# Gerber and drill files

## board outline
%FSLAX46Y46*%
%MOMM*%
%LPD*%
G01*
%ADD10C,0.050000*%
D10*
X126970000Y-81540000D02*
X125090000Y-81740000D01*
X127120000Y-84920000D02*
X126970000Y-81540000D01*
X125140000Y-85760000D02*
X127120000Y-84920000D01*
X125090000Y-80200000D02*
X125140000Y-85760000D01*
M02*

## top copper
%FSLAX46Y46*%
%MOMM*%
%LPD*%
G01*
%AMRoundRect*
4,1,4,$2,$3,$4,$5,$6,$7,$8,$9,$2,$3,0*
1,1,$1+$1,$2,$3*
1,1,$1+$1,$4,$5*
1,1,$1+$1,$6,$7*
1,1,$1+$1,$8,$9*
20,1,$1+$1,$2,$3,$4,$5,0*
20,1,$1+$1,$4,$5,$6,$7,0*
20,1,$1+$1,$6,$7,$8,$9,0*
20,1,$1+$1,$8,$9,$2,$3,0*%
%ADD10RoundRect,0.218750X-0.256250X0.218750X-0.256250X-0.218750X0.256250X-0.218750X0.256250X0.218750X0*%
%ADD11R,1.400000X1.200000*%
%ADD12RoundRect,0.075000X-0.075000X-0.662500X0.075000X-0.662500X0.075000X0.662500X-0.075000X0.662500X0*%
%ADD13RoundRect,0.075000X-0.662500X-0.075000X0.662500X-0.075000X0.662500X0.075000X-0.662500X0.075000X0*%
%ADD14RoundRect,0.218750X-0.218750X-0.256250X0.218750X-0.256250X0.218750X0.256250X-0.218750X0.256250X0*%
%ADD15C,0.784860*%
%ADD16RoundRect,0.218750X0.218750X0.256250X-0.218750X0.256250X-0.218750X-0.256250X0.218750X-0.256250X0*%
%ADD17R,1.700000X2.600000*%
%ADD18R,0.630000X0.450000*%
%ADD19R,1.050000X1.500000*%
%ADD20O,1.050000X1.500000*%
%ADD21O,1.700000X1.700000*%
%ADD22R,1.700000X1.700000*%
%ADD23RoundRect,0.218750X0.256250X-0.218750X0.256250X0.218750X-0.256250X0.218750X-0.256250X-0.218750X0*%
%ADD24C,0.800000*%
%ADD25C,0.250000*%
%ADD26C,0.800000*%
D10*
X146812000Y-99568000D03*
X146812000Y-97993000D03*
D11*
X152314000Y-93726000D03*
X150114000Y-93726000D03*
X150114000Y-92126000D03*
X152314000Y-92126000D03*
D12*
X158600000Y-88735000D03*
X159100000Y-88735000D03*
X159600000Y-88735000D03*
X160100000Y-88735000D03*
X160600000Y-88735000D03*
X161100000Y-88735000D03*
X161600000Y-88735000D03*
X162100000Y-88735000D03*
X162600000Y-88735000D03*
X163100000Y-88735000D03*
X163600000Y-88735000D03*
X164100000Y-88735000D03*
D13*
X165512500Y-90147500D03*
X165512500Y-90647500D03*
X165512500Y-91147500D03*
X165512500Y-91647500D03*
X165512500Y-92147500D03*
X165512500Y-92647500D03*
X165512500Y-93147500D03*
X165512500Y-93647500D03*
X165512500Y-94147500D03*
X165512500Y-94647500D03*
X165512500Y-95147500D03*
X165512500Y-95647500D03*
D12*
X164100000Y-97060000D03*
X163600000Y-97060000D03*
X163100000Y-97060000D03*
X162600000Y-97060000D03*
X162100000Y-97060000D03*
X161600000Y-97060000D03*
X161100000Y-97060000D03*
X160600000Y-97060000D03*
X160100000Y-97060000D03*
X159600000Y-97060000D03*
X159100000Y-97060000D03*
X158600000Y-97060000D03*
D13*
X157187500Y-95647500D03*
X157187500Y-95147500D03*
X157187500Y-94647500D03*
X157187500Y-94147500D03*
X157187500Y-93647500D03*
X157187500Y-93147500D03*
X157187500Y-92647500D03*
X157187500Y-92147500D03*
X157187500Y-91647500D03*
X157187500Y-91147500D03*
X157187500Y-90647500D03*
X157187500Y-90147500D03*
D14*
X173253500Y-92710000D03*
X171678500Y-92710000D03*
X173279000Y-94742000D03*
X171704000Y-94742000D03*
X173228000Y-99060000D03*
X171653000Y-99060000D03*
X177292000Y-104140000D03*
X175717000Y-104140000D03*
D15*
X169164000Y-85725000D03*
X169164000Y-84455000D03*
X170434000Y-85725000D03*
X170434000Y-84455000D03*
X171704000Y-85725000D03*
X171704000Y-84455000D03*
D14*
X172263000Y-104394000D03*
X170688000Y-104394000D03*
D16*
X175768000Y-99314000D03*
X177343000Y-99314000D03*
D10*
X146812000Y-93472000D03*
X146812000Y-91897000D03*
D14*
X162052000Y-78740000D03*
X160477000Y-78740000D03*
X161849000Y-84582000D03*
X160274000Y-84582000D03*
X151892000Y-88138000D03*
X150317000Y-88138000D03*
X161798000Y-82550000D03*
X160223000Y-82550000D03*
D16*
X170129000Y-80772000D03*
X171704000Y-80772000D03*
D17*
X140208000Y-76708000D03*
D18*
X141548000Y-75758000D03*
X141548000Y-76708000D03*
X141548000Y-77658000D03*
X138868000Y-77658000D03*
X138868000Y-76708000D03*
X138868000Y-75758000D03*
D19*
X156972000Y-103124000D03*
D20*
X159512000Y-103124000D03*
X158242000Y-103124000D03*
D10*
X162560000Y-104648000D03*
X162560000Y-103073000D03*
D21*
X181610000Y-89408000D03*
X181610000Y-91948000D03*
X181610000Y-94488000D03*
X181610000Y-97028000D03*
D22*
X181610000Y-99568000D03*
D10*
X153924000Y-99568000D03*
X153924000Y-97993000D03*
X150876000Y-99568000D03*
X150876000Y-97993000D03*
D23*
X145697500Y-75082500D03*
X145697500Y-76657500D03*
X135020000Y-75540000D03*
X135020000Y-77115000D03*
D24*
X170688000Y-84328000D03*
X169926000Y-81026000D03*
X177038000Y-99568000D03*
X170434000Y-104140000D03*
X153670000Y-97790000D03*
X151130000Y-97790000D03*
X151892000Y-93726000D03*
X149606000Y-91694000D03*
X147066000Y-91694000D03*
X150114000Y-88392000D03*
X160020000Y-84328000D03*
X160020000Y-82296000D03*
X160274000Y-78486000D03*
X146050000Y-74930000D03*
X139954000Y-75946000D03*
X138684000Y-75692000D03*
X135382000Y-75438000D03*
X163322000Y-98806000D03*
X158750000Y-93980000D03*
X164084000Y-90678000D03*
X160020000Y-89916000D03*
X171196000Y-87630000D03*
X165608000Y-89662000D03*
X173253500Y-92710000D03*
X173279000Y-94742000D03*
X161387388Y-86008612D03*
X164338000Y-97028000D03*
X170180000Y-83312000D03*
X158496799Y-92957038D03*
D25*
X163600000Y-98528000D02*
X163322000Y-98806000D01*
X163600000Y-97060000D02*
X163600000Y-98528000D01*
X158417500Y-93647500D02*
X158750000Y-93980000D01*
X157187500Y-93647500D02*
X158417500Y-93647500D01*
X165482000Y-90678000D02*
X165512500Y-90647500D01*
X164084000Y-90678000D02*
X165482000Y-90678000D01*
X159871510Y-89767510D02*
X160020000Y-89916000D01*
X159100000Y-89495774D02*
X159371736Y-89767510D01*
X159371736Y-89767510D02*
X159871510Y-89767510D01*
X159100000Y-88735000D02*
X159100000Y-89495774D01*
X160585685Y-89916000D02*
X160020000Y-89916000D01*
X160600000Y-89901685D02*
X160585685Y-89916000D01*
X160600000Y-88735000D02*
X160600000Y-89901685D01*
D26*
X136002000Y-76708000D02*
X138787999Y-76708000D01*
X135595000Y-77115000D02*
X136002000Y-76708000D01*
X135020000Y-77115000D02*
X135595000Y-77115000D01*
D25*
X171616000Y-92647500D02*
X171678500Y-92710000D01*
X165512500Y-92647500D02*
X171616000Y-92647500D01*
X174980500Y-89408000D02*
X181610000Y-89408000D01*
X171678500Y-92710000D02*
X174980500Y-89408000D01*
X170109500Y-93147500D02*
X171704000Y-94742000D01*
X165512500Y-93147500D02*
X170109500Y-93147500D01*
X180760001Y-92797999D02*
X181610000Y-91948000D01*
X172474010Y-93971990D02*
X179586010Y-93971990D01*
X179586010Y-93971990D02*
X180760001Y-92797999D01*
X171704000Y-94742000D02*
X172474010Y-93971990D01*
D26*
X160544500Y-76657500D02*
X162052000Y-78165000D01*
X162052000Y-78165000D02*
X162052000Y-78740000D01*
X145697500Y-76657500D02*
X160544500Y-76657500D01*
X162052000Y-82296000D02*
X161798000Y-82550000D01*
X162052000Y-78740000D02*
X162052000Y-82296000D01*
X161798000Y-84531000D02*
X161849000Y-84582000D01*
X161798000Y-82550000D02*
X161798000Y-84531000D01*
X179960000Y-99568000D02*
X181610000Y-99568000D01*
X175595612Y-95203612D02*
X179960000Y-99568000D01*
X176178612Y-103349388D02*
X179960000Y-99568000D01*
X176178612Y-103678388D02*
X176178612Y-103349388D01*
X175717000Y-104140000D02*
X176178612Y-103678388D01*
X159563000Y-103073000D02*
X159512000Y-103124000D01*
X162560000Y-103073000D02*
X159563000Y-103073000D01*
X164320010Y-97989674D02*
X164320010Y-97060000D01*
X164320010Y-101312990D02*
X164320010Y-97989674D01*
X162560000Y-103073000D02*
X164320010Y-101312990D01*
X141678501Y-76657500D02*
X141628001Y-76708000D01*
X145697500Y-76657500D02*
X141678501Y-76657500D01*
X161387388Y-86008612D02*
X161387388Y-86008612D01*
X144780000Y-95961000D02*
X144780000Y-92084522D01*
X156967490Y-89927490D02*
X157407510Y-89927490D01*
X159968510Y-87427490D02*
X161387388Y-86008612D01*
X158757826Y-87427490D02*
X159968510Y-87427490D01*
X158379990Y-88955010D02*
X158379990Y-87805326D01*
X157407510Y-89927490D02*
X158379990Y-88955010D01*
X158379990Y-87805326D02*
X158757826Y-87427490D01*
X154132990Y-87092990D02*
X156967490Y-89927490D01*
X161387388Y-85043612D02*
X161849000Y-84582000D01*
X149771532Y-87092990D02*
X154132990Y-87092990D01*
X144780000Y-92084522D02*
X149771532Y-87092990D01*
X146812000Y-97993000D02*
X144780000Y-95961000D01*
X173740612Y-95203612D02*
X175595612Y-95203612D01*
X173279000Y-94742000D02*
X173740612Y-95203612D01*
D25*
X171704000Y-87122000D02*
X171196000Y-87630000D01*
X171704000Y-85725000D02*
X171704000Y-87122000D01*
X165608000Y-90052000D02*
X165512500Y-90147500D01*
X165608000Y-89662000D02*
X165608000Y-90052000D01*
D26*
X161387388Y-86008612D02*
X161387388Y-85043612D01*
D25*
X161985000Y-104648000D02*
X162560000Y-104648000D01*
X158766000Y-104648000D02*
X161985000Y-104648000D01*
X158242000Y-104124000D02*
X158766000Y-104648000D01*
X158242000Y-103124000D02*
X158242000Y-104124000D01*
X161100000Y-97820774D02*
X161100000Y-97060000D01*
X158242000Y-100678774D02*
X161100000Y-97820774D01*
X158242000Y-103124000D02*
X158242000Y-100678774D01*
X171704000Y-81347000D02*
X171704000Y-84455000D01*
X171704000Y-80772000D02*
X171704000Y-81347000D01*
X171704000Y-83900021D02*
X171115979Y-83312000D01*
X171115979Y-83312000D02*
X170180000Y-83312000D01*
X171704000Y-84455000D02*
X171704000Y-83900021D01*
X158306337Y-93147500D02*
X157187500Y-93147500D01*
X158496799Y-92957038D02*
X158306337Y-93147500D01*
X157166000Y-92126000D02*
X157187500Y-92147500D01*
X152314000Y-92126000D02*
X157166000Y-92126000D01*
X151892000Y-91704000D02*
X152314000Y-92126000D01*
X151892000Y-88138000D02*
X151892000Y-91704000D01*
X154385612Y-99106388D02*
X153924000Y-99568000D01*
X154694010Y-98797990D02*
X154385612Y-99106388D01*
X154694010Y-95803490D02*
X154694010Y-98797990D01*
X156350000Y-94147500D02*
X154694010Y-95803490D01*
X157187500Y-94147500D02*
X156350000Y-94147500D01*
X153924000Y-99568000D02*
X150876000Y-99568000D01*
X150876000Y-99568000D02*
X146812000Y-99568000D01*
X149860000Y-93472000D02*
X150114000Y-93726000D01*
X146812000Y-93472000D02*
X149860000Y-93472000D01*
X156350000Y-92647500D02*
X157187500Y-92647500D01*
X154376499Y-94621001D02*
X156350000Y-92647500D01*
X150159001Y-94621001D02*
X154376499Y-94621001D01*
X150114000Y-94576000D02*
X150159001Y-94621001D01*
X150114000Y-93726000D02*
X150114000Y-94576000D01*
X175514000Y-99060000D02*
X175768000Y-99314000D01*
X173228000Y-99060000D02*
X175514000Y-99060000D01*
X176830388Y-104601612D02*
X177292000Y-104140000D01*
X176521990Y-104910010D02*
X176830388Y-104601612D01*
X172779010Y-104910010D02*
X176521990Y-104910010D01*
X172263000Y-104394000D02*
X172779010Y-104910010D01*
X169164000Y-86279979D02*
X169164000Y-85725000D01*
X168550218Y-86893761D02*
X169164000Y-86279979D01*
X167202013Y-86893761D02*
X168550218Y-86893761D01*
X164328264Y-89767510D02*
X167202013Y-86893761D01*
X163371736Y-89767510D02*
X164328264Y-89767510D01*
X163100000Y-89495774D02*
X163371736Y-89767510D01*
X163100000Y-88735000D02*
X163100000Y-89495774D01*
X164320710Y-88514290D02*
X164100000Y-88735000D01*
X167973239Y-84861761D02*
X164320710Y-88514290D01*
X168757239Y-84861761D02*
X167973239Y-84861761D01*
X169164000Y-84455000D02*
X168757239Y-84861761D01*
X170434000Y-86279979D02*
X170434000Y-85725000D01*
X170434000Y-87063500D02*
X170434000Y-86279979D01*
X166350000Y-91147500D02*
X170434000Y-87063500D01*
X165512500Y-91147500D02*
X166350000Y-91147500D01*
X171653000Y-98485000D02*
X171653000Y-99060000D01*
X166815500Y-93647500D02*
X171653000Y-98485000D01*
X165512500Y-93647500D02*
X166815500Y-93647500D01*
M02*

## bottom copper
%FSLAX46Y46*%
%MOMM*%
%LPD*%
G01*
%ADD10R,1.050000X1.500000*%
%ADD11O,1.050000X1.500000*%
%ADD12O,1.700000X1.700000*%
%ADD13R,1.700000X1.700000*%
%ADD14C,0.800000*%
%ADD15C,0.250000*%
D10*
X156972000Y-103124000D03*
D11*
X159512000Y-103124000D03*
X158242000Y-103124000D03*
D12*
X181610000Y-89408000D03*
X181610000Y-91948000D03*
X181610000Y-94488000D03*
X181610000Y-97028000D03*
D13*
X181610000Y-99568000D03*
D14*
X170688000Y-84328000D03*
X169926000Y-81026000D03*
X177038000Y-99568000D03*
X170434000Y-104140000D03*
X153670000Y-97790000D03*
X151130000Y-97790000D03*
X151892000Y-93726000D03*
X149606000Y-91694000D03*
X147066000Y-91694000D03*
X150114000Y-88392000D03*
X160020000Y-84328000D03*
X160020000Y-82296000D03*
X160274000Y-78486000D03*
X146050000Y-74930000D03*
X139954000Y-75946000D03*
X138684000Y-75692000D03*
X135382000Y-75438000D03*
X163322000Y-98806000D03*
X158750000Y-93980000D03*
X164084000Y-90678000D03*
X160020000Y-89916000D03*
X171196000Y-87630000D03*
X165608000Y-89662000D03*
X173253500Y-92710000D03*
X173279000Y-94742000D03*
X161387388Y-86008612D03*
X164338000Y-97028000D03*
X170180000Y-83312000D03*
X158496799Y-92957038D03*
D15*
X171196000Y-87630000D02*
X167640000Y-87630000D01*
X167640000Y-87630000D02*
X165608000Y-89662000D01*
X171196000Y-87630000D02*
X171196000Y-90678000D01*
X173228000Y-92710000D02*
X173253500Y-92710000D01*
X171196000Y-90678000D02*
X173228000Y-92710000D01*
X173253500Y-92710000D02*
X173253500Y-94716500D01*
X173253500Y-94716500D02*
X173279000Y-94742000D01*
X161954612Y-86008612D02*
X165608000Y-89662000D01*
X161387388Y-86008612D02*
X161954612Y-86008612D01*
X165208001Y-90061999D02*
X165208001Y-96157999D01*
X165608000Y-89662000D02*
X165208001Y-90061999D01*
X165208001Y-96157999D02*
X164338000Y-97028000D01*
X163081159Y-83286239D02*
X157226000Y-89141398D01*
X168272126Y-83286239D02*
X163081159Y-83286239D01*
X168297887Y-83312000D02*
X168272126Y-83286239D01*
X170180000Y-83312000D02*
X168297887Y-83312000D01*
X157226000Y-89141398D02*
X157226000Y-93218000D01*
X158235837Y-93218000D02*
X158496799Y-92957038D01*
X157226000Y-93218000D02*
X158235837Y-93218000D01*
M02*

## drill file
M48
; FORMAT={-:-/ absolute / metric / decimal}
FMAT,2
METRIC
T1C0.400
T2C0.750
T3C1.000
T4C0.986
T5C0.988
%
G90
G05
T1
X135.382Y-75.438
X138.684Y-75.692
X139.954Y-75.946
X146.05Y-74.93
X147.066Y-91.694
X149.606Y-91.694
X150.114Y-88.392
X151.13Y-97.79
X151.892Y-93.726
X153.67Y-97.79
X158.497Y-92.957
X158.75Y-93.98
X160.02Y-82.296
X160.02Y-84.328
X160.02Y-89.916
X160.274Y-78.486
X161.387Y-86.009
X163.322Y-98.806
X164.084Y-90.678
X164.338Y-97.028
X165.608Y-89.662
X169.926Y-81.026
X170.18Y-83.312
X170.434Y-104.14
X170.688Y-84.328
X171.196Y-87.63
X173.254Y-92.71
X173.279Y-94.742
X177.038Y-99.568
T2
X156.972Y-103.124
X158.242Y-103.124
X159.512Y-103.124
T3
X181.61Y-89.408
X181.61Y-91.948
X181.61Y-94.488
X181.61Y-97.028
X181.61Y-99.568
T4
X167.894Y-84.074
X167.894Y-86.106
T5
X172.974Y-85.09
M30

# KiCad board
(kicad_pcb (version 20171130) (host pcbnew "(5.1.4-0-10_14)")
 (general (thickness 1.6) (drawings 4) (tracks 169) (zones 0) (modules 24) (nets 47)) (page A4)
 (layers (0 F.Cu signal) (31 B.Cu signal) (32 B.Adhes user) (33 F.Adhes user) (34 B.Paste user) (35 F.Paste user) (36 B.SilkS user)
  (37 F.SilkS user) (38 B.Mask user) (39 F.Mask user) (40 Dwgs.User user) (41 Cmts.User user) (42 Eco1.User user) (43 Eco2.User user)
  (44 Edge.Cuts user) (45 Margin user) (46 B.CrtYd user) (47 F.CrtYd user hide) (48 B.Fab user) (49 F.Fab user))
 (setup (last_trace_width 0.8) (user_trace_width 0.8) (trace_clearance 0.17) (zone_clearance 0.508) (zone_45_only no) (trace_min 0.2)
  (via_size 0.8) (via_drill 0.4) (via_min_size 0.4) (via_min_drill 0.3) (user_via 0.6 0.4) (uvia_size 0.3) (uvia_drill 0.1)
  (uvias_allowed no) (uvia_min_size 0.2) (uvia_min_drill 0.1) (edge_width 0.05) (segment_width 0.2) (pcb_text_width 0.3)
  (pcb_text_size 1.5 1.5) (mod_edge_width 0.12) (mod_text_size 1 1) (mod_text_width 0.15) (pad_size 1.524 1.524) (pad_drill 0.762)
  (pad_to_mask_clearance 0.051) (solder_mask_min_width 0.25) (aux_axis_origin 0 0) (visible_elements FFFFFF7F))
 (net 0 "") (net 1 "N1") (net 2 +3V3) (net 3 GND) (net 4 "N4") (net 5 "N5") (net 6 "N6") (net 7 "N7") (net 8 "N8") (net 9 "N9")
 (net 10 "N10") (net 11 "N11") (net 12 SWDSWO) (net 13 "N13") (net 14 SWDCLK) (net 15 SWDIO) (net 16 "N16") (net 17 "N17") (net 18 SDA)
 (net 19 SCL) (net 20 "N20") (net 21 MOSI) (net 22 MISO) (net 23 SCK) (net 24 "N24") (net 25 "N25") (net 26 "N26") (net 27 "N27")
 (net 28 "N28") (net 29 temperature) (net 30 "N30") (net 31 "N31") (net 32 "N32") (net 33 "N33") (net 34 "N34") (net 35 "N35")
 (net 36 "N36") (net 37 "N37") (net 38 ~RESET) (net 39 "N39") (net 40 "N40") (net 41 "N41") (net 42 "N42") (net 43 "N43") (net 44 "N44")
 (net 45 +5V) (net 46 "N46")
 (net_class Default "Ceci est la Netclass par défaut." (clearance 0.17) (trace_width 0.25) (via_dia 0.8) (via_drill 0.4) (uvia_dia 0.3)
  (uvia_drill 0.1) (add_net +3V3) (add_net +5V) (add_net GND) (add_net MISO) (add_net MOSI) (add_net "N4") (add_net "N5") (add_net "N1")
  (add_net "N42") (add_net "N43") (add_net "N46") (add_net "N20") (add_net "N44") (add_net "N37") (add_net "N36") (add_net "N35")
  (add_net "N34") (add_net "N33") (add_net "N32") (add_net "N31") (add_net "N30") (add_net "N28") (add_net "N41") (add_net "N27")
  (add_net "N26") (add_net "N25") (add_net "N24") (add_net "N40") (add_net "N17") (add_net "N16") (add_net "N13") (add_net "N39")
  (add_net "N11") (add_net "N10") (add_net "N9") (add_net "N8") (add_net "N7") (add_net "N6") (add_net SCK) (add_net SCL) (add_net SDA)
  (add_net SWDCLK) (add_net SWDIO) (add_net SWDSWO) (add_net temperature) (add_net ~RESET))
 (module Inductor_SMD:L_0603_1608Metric (layer F.Cu) (at 146.812 98.7805 270)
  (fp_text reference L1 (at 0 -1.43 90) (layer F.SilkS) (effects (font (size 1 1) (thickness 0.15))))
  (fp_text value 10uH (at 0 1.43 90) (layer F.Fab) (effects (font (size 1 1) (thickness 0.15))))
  (pad 2 smd roundrect (at 0.7875 0 270) (size 0.875 0.95) (layers F.Cu F.Paste F.Mask) (roundrect_rratio 0.25) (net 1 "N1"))
  (pad 1 smd roundrect (at -0.7875 0 270) (size 0.875 0.95) (layers F.Cu F.Paste F.Mask) (roundrect_rratio 0.25) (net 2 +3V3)))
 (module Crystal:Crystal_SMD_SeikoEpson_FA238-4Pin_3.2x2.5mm (layer F.Cu) (at 151.214 92.926 180)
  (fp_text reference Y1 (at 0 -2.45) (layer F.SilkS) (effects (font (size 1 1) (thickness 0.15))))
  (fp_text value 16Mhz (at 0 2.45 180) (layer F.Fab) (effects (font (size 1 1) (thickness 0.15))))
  (pad 4 smd rect (at -1.1 -0.8 180) (size 1.4 1.2) (layers F.Cu F.Paste F.Mask) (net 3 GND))
  (pad 3 smd rect (at 1.1 -0.8 180) (size 1.4 1.2) (layers F.Cu F.Paste F.Mask) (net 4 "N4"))
  (pad 2 smd rect (at 1.1 0.8 180) (size 1.4 1.2) (layers F.Cu F.Paste F.Mask) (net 3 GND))
  (pad 1 smd rect (at -1.1 0.8 180) (size 1.4 1.2) (layers F.Cu F.Paste F.Mask) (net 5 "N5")))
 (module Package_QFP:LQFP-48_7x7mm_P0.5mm (layer F.Cu) (at 161.35 92.8975)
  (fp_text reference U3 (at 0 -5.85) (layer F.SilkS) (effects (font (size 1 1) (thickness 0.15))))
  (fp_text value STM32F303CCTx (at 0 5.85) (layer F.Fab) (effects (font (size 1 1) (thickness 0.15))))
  (pad 48 smd roundrect (at -2.75 -4.1625) (size 0.3 1.475) (layers F.Cu F.Paste F.Mask) (roundrect_rratio 0.25) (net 2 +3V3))
  (pad 47 smd roundrect (at -2.25 -4.1625) (size 0.3 1.475) (layers F.Cu F.Paste F.Mask) (roundrect_rratio 0.25) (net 3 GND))
  (pad 46 smd roundrect (at -1.75 -4.1625) (size 0.3 1.475) (layers F.Cu F.Paste F.Mask) (roundrect_rratio 0.25) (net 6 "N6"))
  (pad 45 smd roundrect (at -1.25 -4.1625) (size 0.3 1.475) (layers F.Cu F.Paste F.Mask) (roundrect_rratio 0.25) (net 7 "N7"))
  (pad 44 smd roundrect (at -0.75 -4.1625) (size 0.3 1.475) (layers F.Cu F.Paste F.Mask) (roundrect_rratio 0.25) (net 3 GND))
  (pad 43 smd roundrect (at -0.25 -4.1625) (size 0.3 1.475) (layers F.Cu F.Paste F.Mask) (roundrect_rratio 0.25) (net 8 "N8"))
  (pad 42 smd roundrect (at 0.25 -4.1625) (size 0.3 1.475) (layers F.Cu F.Paste F.Mask) (roundrect_rratio 0.25) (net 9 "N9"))
  (pad 41 smd roundrect (at 0.75 -4.1625) (size 0.3 1.475) (layers F.Cu F.Paste F.Mask) (roundrect_rratio 0.25) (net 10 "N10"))
  (pad 40 smd roundrect (at 1.25 -4.1625) (size 0.3 1.475) (layers F.Cu F.Paste F.Mask) (roundrect_rratio 0.25) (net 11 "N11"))
  (pad 39 smd roundrect (at 1.75 -4.1625) (size 0.3 1.475) (layers F.Cu F.Paste F.Mask) (roundrect_rratio 0.25) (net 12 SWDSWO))
  (pad 38 smd roundrect (at 2.25 -4.1625) (size 0.3 1.475) (layers F.Cu F.Paste F.Mask) (roundrect_rratio 0.25) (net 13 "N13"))
  (pad 37 smd roundrect (at 2.75 -4.1625) (size 0.3 1.475) (layers F.Cu F.Paste F.Mask) (roundrect_rratio 0.25) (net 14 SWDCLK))
  (pad 36 smd roundrect (at 4.1625 -2.75) (size 1.475 0.3) (layers F.Cu F.Paste F.Mask) (roundrect_rratio 0.25) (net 2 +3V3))
  (pad 35 smd roundrect (at 4.1625 -2.25) (size 1.475 0.3) (layers F.Cu F.Paste F.Mask) (roundrect_rratio 0.25) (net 3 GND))
  (pad 34 smd roundrect (at 4.1625 -1.75) (size 1.475 0.3) (layers F.Cu F.Paste F.Mask) (roundrect_rratio 0.25) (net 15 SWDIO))
  (pad 33 smd roundrect (at 4.1625 -1.25) (size 1.475 0.3) (layers F.Cu F.Paste F.Mask) (roundrect_rratio 0.25) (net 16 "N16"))
  (pad 32 smd roundrect (at 4.1625 -0.75) (size 1.475 0.3) (layers F.Cu F.Paste F.Mask) (roundrect_rratio 0.25) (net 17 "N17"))
  (pad 31 smd roundrect (at 4.1625 -0.25) (size 1.475 0.3) (layers F.Cu F.Paste F.Mask) (roundrect_rratio 0.25) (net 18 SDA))
  (pad 30 smd roundrect (at 4.1625 0.25) (size 1.475 0.3) (layers F.Cu F.Paste F.Mask) (roundrect_rratio 0.25) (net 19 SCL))
  (pad 29 smd roundrect (at 4.1625 0.75) (size 1.475 0.3) (layers F.Cu F.Paste F.Mask) (roundrect_rratio 0.25) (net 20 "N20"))
  (pad 28 smd roundrect (at 4.1625 1.25) (size 1.475 0.3) (layers F.Cu F.Paste F.Mask) (roundrect_rratio 0.25) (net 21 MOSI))
  (pad 27 smd roundrect (at 4.1625 1.75) (size 1.475 0.3) (layers F.Cu F.Paste F.Mask) (roundrect_rratio 0.25) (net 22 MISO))
  (pad 26 smd roundrect (at 4.1625 2.25) (size 1.475 0.3) (layers F.Cu F.Paste F.Mask) (roundrect_rratio 0.25) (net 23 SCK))
  (pad 25 smd roundrect (at 4.1625 2.75) (size 1.475 0.3) (layers F.Cu F.Paste F.Mask) (roundrect_rratio 0.25) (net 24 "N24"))
  (pad 24 smd roundrect (at 2.75 4.1625) (size 0.3 1.475) (layers F.Cu F.Paste F.Mask) (roundrect_rratio 0.25) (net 2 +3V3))
  (pad 23 smd roundrect (at 2.25 4.1625) (size 0.3 1.475) (layers F.Cu F.Paste F.Mask) (roundrect_rratio 0.25) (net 3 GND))
  (pad 22 smd roundrect (at 1.75 4.1625) (size 0.3 1.475) (layers F.Cu F.Paste F.Mask) (roundrect_rratio 0.25) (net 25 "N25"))
  (pad 21 smd roundrect (at 1.25 4.1625) (size 0.3 1.475) (layers F.Cu F.Paste F.Mask) (roundrect_rratio 0.25) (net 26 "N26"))
  (pad 20 smd roundrect (at 0.75 4.1625) (size 0.3 1.475) (layers F.Cu F.Paste F.Mask) (roundrect_rratio 0.25) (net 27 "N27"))
  (pad 19 smd roundrect (at 0.25 4.1625) (size 0.3 1.475) (layers F.Cu F.Paste F.Mask) (roundrect_rratio 0.25) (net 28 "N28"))
  (pad 18 smd roundrect (at -0.25 4.1625) (size 0.3 1.475) (layers F.Cu F.Paste F.Mask) (roundrect_rratio 0.25) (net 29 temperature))
  (pad 17 smd roundrect (at -0.75 4.1625) (size 0.3 1.475) (layers F.Cu F.Paste F.Mask) (roundrect_rratio 0.25) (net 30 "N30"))
  (pad 16 smd roundrect (at -1.25 4.1625) (size 0.3 1.475) (layers F.Cu F.Paste F.Mask) (roundrect_rratio 0.25) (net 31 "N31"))
  (pad 15 smd roundrect (at -1.75 4.1625) (size 0.3 1.475) (layers F.Cu F.Paste F.Mask) (roundrect_rratio 0.25) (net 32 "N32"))
  (pad 14 smd roundrect (at -2.25 4.1625) (size 0.3 1.475) (layers F.Cu F.Paste F.Mask) (roundrect_rratio 0.25) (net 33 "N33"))
  (pad 13 smd roundrect (at -2.75 4.1625) (size 0.3 1.475) (layers F.Cu F.Paste F.Mask) (roundrect_rratio 0.25) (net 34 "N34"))
  (pad 12 smd roundrect (at -4.1625 2.75) (size 1.475 0.3) (layers F.Cu F.Paste F.Mask) (roundrect_rratio 0.25) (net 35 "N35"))
  (pad 11 smd roundrect (at -4.1625 2.25) (size 1.475 0.3) (layers F.Cu F.Paste F.Mask) (roundrect_rratio 0.25) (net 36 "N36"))
  (pad 10 smd roundrect (at -4.1625 1.75) (size 1.475 0.3) (layers F.Cu F.Paste F.Mask) (roundrect_rratio 0.25) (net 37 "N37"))
  (pad 9 smd roundrect (at -4.1625 1.25) (size 1.475 0.3) (layers F.Cu F.Paste F.Mask) (roundrect_rratio 0.25) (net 1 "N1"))
  (pad 8 smd roundrect (at -4.1625 0.75) (size 1.475 0.3) (layers F.Cu F.Paste F.Mask) (roundrect_rratio 0.25) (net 3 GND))
  (pad 7 smd roundrect (at -4.1625 0.25) (size 1.475 0.3) (layers F.Cu F.Paste F.Mask) (roundrect_rratio 0.25) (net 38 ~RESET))
  (pad 6 smd roundrect (at -4.1625 -0.25) (size 1.475 0.3) (layers F.Cu F.Paste F.Mask) (roundrect_rratio 0.25) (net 4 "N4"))
  (pad 5 smd roundrect (at -4.1625 -0.75) (size 1.475 0.3) (layers F.Cu F.Paste F.Mask) (roundrect_rratio 0.25) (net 5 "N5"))
  (pad 4 smd roundrect (at -4.1625 -1.25) (size 1.475 0.3) (layers F.Cu F.Paste F.Mask) (roundrect_rratio 0.25) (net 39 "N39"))
  (pad 3 smd roundrect (at -4.1625 -1.75) (size 1.475 0.3) (layers F.Cu F.Paste F.Mask) (roundrect_rratio 0.25) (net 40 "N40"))
  (pad 2 smd roundrect (at -4.1625 -2.25) (size 1.475 0.3) (layers F.Cu F.Paste F.Mask) (roundrect_rratio 0.25) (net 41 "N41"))
  (pad 1 smd roundrect (at -4.1625 -2.75) (size 1.475 0.3) (layers F.Cu F.Paste F.Mask) (roundrect_rratio 0.25) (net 2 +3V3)))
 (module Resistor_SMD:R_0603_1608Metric (layer F.Cu) (at 172.466 92.71)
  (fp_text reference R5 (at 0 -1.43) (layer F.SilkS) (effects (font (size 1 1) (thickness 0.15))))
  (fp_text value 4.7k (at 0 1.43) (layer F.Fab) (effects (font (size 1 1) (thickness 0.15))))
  (pad 2 smd roundrect (at 0.7875 0) (size 0.875 0.95) (layers F.Cu F.Paste F.Mask) (roundrect_rratio 0.25) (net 2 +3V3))
  (pad 1 smd roundrect (at -0.7875 0) (size 0.875 0.95) (layers F.Cu F.Paste F.Mask) (roundrect_rratio 0.25) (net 18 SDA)))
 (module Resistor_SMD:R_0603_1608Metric (layer F.Cu) (at 172.4915 94.742)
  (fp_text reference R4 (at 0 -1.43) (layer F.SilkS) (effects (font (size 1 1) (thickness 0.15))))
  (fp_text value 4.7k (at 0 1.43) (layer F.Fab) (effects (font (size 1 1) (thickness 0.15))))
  (pad 2 smd roundrect (at 0.7875 0) (size 0.875 0.95) (layers F.Cu F.Paste F.Mask) (roundrect_rratio 0.25) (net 2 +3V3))
  (pad 1 smd roundrect (at -0.7875 0) (size 0.875 0.95) (layers F.Cu F.Paste F.Mask) (roundrect_rratio 0.25) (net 19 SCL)))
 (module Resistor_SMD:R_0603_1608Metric (layer F.Cu) (at 172.4405 99.06)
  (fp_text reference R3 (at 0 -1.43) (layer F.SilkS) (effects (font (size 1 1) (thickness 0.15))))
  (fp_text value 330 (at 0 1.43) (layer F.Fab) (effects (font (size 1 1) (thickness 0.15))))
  (pad 2 smd roundrect (at 0.7875 0) (size 0.875 0.95) (layers F.Cu F.Paste F.Mask) (roundrect_rratio 0.25) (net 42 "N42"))
  (pad 1 smd roundrect (at -0.7875 0) (size 0.875 0.95) (layers F.Cu F.Paste F.Mask) (roundrect_rratio 0.25) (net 20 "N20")))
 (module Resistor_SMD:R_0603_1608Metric (layer F.Cu) (at 176.5045 104.14)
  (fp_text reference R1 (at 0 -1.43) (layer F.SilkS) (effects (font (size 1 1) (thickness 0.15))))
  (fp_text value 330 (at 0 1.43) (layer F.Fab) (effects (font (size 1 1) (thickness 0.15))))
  (pad 2 smd roundrect (at 0.7875 0) (size 0.875 0.95) (layers F.Cu F.Paste F.Mask) (roundrect_rratio 0.25) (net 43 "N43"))
  (pad 1 smd roundrect (at -0.7875 0) (size 0.875 0.95) (layers F.Cu F.Paste F.Mask) (roundrect_rratio 0.25) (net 2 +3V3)))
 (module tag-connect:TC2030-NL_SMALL (layer F.Cu) (at 170.434 85.09 180) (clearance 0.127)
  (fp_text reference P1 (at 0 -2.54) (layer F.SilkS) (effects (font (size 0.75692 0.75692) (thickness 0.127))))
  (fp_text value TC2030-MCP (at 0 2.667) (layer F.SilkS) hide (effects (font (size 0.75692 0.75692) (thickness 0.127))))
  (pad "" np_thru_hole circle (at 2.54 1.016 180) (size 0.98552 0.98552) (drill 0.98552) (layers *.Cu *.Mask F.SilkS))
  (pad "" np_thru_hole circle (at 2.54 -1.016 180) (size 0.98552 0.98552) (drill 0.98552) (layers *.Cu *.Mask F.SilkS))
  (pad "" np_thru_hole circle (at -2.54 0 180) (size 0.98806 0.98806) (drill 0.98806) (layers *.Cu *.Mask F.SilkS))
  (pad 6 connect circle (at 1.27 -0.635 180) (size 0.78486 0.78486) (layers F.Cu F.Mask) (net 12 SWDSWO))
  (pad 5 connect circle (at 1.27 0.635 180) (size 0.78486 0.78486) (layers F.Cu F.Mask) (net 14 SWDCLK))
  (pad 4 connect circle (at 0 -0.635 180) (size 0.78486 0.78486) (layers F.Cu F.Mask) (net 15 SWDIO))
  (pad 3 connect circle (at 0 0.635 180) (size 0.78486 0.78486) (layers F.Cu F.Mask) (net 3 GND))
  (pad 2 connect circle (at -1.27 -0.635 180) (size 0.78486 0.78486) (layers F.Cu F.Mask) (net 2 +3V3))
  (pad 1 connect circle (at -1.27 0.635 180) (size 0.78486 0.78486) (layers F.Cu F.Mask) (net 38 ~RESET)))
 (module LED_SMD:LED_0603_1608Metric (layer F.Cu) (at 171.4755 104.394)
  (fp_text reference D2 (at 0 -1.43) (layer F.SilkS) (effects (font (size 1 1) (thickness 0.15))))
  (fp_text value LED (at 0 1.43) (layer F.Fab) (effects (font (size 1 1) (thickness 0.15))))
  (pad 2 smd roundrect (at 0.7875 0) (size 0.875 0.95) (layers F.Cu F.Paste F.Mask) (roundrect_rratio 0.25) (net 43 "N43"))
  (pad 1 smd roundrect (at -0.7875 0) (size 0.875 0.95) (layers F.Cu F.Paste F.Mask) (roundrect_rratio 0.25) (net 3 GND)))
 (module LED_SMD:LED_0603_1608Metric (layer F.Cu) (at 176.5555 99.314 180)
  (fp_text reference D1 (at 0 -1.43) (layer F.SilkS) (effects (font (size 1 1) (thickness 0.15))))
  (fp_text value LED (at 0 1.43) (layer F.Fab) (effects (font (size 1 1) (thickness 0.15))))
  (pad 2 smd roundrect (at 0.7875 0 180) (size 0.875 0.95) (layers F.Cu F.Paste F.Mask) (roundrect_rratio 0.25) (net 42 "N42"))
  (pad 1 smd roundrect (at -0.7875 0 180) (size 0.875 0.95) (layers F.Cu F.Paste F.Mask) (roundrect_rratio 0.25) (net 3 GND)))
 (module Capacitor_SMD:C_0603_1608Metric (layer F.Cu) (at 146.812 92.6845 270)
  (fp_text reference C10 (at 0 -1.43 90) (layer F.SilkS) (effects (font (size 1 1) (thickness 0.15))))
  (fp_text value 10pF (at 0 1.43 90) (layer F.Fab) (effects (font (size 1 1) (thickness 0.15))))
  (pad 2 smd roundrect (at 0.7875 0 270) (size 0.875 0.95) (layers F.Cu F.Paste F.Mask) (roundrect_rratio 0.25) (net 4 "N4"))
  (pad 1 smd roundrect (at -0.7875 0 270) (size 0.875 0.95) (layers F.Cu F.Paste F.Mask) (roundrect_rratio 0.25) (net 3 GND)))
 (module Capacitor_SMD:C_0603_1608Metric (layer F.Cu) (at 161.2645 78.74)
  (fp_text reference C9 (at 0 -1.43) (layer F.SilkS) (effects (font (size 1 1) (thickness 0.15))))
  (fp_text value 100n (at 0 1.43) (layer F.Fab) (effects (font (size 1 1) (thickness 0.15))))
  (pad 2 smd roundrect (at 0.7875 0) (size 0.875 0.95) (layers F.Cu F.Paste F.Mask) (roundrect_rratio 0.25) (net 2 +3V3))
  (pad 1 smd roundrect (at -0.7875 0) (size 0.875 0.95) (layers F.Cu F.Paste F.Mask) (roundrect_rratio 0.25) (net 3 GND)))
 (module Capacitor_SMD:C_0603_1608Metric (layer F.Cu) (at 161.0615 84.582)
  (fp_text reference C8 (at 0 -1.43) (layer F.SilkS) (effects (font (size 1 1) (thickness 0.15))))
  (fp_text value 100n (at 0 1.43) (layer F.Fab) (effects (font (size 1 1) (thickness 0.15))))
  (pad 2 smd roundrect (at 0.7875 0) (size 0.875 0.95) (layers F.Cu F.Paste F.Mask) (roundrect_rratio 0.25) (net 2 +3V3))
  (pad 1 smd roundrect (at -0.7875 0) (size 0.875 0.95) (layers F.Cu F.Paste F.Mask) (roundrect_rratio 0.25) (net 3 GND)))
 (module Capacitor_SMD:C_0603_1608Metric (layer F.Cu) (at 151.1045 88.138)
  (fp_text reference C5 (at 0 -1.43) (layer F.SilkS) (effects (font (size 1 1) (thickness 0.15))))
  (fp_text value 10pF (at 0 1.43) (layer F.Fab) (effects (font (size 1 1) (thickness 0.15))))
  (pad 2 smd roundrect (at 0.7875 0) (size 0.875 0.95) (layers F.Cu F.Paste F.Mask) (roundrect_rratio 0.25) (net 5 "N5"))
  (pad 1 smd roundrect (at -0.7875 0) (size 0.875 0.95) (layers F.Cu F.Paste F.Mask) (roundrect_rratio 0.25) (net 3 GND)))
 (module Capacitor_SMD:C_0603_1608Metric (layer F.Cu) (at 161.0105 82.55)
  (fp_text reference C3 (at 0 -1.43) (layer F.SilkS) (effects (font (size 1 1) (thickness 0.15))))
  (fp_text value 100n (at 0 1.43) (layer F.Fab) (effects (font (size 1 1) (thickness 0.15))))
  (pad 2 smd roundrect (at 0.7875 0) (size 0.875 0.95) (layers F.Cu F.Paste F.Mask) (roundrect_rratio 0.25) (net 2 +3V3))
  (pad 1 smd roundrect (at -0.7875 0) (size 0.875 0.95) (layers F.Cu F.Paste F.Mask) (roundrect_rratio 0.25) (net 3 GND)))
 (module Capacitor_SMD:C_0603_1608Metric (layer F.Cu) (at 170.9165 80.772 180)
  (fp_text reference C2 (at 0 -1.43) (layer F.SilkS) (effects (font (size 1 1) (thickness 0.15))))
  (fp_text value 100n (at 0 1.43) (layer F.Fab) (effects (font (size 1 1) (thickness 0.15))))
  (pad 2 smd roundrect (at 0.7875 0 180) (size 0.875 0.95) (layers F.Cu F.Paste F.Mask) (roundrect_rratio 0.25) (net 3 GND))
  (pad 1 smd roundrect (at -0.7875 0 180) (size 0.875 0.95) (layers F.Cu F.Paste F.Mask) (roundrect_rratio 0.25) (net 38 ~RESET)))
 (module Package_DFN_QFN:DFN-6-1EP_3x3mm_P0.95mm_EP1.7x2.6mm (layer F.Cu) (at 140.208 76.708)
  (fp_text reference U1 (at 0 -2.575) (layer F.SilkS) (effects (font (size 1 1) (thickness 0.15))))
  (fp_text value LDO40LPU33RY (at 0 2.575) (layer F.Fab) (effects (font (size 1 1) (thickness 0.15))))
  (pad "" smd rect (at -0.425 -0.866) (size 0.66 0.73) (layers F.Paste))
  (pad "" smd rect (at 0.425 -0.866) (size 0.66 0.73) (layers F.Paste))
  (pad "" smd rect (at -0.425 0) (size 0.66 0.73) (layers F.Paste))
  (pad "" smd rect (at 0.425 0) (size 0.66 0.73) (layers F.Paste))
  (pad "" smd rect (at 0.425 0.866) (size 0.66 0.73) (layers F.Paste))
  (pad 7 smd rect (at 0 0) (size 1.7 2.6) (layers F.Cu F.Mask) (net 3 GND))
  (pad "" smd rect (at -0.425 0.866) (size 0.66 0.73) (layers F.Paste))
  (pad 6 smd rect (at 1.34 -0.95) (size 0.63 0.45) (layers F.Cu F.Paste F.Mask) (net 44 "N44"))
  (pad 5 smd rect (at 1.34 0) (size 0.63 0.45) (layers F.Cu F.Paste F.Mask) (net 2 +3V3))
  (pad 4 smd rect (at 1.34 0.95) (size 0.63 0.45) (layers F.Cu F.Paste F.Mask) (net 2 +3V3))
  (pad 3 smd rect (at -1.34 0.95) (size 0.63 0.45) (layers F.Cu F.Paste F.Mask) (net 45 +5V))
  (pad 2 smd rect (at -1.34 0) (size 0.63 0.45) (layers F.Cu F.Paste F.Mask) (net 45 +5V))
  (pad 1 smd rect (at -1.34 -0.95) (size 0.63 0.45) (layers F.Cu F.Paste F.Mask) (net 3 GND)))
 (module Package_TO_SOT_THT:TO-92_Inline (layer F.Cu) (at 156.972 103.124)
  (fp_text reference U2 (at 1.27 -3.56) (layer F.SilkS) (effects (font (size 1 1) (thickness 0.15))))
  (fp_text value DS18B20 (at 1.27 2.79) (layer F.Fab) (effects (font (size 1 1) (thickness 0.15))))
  (pad 1 thru_hole rect (at 0 0) (size 1.05 1.5) (drill 0.75) (layers *.Cu *.Mask) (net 3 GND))
  (pad 3 thru_hole oval (at 2.54 0) (size 1.05 1.5) (drill 0.75) (layers *.Cu *.Mask) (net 2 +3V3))
  (pad 2 thru_hole oval (at 1.27 0) (size 1.05 1.5) (drill 0.75) (layers *.Cu *.Mask) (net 29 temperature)))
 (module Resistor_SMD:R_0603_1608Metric (layer F.Cu) (at 162.56 103.8605 270)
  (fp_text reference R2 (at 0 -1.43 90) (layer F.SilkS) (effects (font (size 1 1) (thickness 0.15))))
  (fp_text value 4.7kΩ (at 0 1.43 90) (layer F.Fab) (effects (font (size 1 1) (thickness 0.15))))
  (pad 2 smd roundrect (at 0.7875 0 270) (size 0.875 0.95) (layers F.Cu F.Paste F.Mask) (roundrect_rratio 0.25) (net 29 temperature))
  (pad 1 smd roundrect (at -0.7875 0 270) (size 0.875 0.95) (layers F.Cu F.Paste F.Mask) (roundrect_rratio 0.25) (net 2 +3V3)))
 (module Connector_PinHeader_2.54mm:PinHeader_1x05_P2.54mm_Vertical (layer F.Cu) (at 181.61 99.568 180)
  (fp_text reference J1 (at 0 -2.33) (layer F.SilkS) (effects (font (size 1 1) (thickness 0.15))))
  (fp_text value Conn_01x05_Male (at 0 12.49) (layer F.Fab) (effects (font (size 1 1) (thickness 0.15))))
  (pad 5 thru_hole oval (at 0 10.16 180) (size 1.7 1.7) (drill 1) (layers *.Cu *.Mask) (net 18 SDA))
  (pad 4 thru_hole oval (at 0 7.62 180) (size 1.7 1.7) (drill 1) (layers *.Cu *.Mask) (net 19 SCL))
  (pad 3 thru_hole oval (at 0 5.08 180) (size 1.7 1.7) (drill 1) (layers *.Cu *.Mask) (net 3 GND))
  (pad 2 thru_hole oval (at 0 2.54 180) (size 1.7 1.7) (drill 1) (layers *.Cu *.Mask) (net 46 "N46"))
  (pad 1 thru_hole rect (at 0 0 180) (size 1.7 1.7) (drill 1) (layers *.Cu *.Mask) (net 2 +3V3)))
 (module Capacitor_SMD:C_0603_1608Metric (layer F.Cu) (at 153.924 98.7805 270)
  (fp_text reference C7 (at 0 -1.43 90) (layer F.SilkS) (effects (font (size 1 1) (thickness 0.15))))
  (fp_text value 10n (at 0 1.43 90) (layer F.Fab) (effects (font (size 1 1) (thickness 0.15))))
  (pad 2 smd roundrect (at 0.7875 0 270) (size 0.875 0.95) (layers F.Cu F.Paste F.Mask) (roundrect_rratio 0.25) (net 1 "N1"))
  (pad 1 smd roundrect (at -0.7875 0 270) (size 0.875 0.95) (layers F.Cu F.Paste F.Mask) (roundrect_rratio 0.25) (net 3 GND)))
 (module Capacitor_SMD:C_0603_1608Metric (layer F.Cu) (at 150.876 98.7805 270)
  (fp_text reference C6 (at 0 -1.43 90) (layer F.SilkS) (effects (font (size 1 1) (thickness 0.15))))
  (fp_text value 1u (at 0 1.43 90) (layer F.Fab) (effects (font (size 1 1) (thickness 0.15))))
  (pad 2 smd roundrect (at 0.7875 0 270) (size 0.875 0.95) (layers F.Cu F.Paste F.Mask) (roundrect_rratio 0.25) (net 1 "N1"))
  (pad 1 smd roundrect (at -0.7875 0 270) (size 0.875 0.95) (layers F.Cu F.Paste F.Mask) (roundrect_rratio 0.25) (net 3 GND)))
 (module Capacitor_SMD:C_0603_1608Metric (layer F.Cu) (at 145.6975 75.87 90)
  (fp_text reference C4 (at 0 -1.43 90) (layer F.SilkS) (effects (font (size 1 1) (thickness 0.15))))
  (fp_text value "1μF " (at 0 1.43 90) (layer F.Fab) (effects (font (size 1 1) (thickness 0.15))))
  (pad 2 smd roundrect (at 0.7875 0 90) (size 0.875 0.95) (layers F.Cu F.Paste F.Mask) (roundrect_rratio 0.25) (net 3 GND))
  (pad 1 smd roundrect (at -0.7875 0 90) (size 0.875 0.95) (layers F.Cu F.Paste F.Mask) (roundrect_rratio 0.25) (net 2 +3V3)))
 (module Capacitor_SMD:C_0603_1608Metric (layer F.Cu) (at 135.02 76.3275 90)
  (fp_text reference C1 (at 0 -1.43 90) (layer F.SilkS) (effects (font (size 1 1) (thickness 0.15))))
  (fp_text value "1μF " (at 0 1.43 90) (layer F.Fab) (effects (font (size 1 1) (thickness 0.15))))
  (pad 2 smd roundrect (at 0.7875 0 90) (size 0.875 0.95) (layers F.Cu F.Paste F.Mask) (roundrect_rratio 0.25) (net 3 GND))
  (pad 1 smd roundrect (at -0.7875 0 90) (size 0.875 0.95) (layers F.Cu F.Paste F.Mask) (roundrect_rratio 0.25) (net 45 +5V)))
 (gr_line (start 126.97 81.54) (end 125.09 81.74) (layer Edge.Cuts) (width 0.05))
 (gr_line (start 127.12 84.92) (end 126.97 81.54) (layer Edge.Cuts) (width 0.05))
 (gr_line (start 125.14 85.76) (end 127.12 84.92) (layer Edge.Cuts) (width 0.05))
 (gr_line (start 125.09 80.2) (end 125.14 85.76) (layer Edge.Cuts) (width 0.05))
 (via (at 170.688 84.328) (size 0.8) (drill 0.4) (layers F.Cu B.Cu) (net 3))
 (via (at 169.926 81.026) (size 0.8) (drill 0.4) (layers F.Cu B.Cu) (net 3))
 (via (at 177.038 99.568) (size 0.8) (drill 0.4) (layers F.Cu B.Cu) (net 3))
 (via (at 170.434 104.14) (size 0.8) (drill 0.4) (layers F.Cu B.Cu) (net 3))
 (via (at 153.67 97.79) (size 0.8) (drill 0.4) (layers F.Cu B.Cu) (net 3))
 (via (at 151.13 97.79) (size 0.8) (drill 0.4) (layers F.Cu B.Cu) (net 3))
 (via (at 151.892 93.726) (size 0.8) (drill 0.4) (layers F.Cu B.Cu) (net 3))
 (via (at 149.606 91.694) (size 0.8) (drill 0.4) (layers F.Cu B.Cu) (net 3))
 (via (at 147.066 91.694) (size 0.8) (drill 0.4) (layers F.Cu B.Cu) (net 3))
 (via (at 150.114 88.392) (size 0.8) (drill 0.4) (layers F.Cu B.Cu) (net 3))
 (via (at 160.02 84.328) (size 0.8) (drill 0.4) (layers F.Cu B.Cu) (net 3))
 (via (at 160.02 82.296) (size 0.8) (drill 0.4) (layers F.Cu B.Cu) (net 3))
 (via (at 160.274 78.486) (size 0.8) (drill 0.4) (layers F.Cu B.Cu) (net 3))
 (via (at 146.05 74.93) (size 0.8) (drill 0.4) (layers F.Cu B.Cu) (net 3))
 (via (at 139.954 75.946) (size 0.8) (drill 0.4) (layers F.Cu B.Cu) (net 3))
 (via (at 138.684 75.692) (size 0.8) (drill 0.4) (layers F.Cu B.Cu) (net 3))
 (via (at 135.382 75.438) (size 0.8) (drill 0.4) (layers F.Cu B.Cu) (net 3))
 (via (at 163.322 98.806) (size 0.8) (drill 0.4) (layers F.Cu B.Cu) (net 3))
 (segment (start 163.6 98.528) (end 163.322 98.806) (width 0.25) (layer F.Cu) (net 3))
 (segment (start 163.6 97.06) (end 163.6 98.528) (width 0.25) (layer F.Cu) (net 3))
 (via (at 158.75 93.98) (size 0.8) (drill 0.4) (layers F.Cu B.Cu) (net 3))
 (segment (start 158.4175 93.6475) (end 158.75 93.98) (width 0.25) (layer F.Cu) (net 3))
 (segment (start 157.1875 93.6475) (end 158.4175 93.6475) (width 0.25) (layer F.Cu) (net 3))
 (via (at 164.084 90.678) (size 0.8) (drill 0.4) (layers F.Cu B.Cu) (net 3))
 (segment (start 165.482 90.678) (end 165.5125 90.6475) (width 0.25) (layer F.Cu) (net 3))
 (segment (start 164.084 90.678) (end 165.482 90.678) (width 0.25) (layer F.Cu) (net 3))
 (via (at 160.02 89.916) (size 0.8) (drill 0.4) (layers F.Cu B.Cu) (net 3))
 (segment (start 159.87151 89.76751) (end 160.02 89.916) (width 0.25) (layer F.Cu) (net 3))
 (segment (start 159.1 89.495774) (end 159.371736 89.76751) (width 0.25) (layer F.Cu) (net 3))
 (segment (start 159.371736 89.76751) (end 159.87151 89.76751) (width 0.25) (layer F.Cu) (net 3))
 (segment (start 159.1 88.735) (end 159.1 89.495774) (width 0.25) (layer F.Cu) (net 3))
 (segment (start 160.585685 89.916) (end 160.02 89.916) (width 0.25) (layer F.Cu) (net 3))
 (segment (start 160.6 89.901685) (end 160.585685 89.916) (width 0.25) (layer F.Cu) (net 3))
 (segment (start 160.6 88.735) (end 160.6 89.901685) (width 0.25) (layer F.Cu) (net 3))
 (segment (start 136.002 76.708) (end 138.787999 76.708) (width 0.8) (layer F.Cu) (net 45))
 (segment (start 135.595 77.115) (end 136.002 76.708) (width 0.8) (layer F.Cu) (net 45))
 (segment (start 135.02 77.115) (end 135.595 77.115) (width 0.8) (layer F.Cu) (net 45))
 (segment (start 171.616 92.6475) (end 171.6785 92.71) (width 0.25) (layer F.Cu) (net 18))
 (segment (start 165.5125 92.6475) (end 171.616 92.6475) (width 0.25) (layer F.Cu) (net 18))
 (segment (start 174.9805 89.408) (end 181.61 89.408) (width 0.25) (layer F.Cu) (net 18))
 (segment (start 171.6785 92.71) (end 174.9805 89.408) (width 0.25) (layer F.Cu) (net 18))
 (segment (start 170.1095 93.1475) (end 171.704 94.742) (width 0.25) (layer F.Cu) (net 19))
 (segment (start 165.5125 93.1475) (end 170.1095 93.1475) (width 0.25) (layer F.Cu) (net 19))
 (segment (start 180.760001 92.797999) (end 181.61 91.948) (width 0.25) (layer F.Cu) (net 19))
 (segment (start 172.47401 93.97199) (end 179.58601 93.97199) (width 0.25) (layer F.Cu) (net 19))
 (segment (start 179.58601 93.97199) (end 180.760001 92.797999) (width 0.25) (layer F.Cu) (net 19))
 (segment (start 171.704 94.742) (end 172.47401 93.97199) (width 0.25) (layer F.Cu) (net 19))
 (segment (start 160.5445 76.6575) (end 162.052 78.165) (width 0.8) (layer F.Cu) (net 2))
 (segment (start 162.052 78.165) (end 162.052 78.74) (width 0.8) (layer F.Cu) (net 2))
 (segment (start 145.6975 76.6575) (end 160.5445 76.6575) (width 0.8) (layer F.Cu) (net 2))
 (segment (start 162.052 82.296) (end 161.798 82.55) (width 0.8) (layer F.Cu) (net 2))
 (segment (start 162.052 78.74) (end 162.052 82.296) (width 0.8) (layer F.Cu) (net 2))
 (segment (start 161.798 84.531) (end 161.849 84.582) (width 0.8) (layer F.Cu) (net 2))
 (segment (start 161.798 82.55) (end 161.798 84.531) (width 0.8) (layer F.Cu) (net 2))
 (segment (start 179.96 99.568) (end 181.61 99.568) (width 0.8) (layer F.Cu) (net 2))
 (segment (start 175.595612 95.203612) (end 179.96 99.568) (width 0.8) (layer F.Cu) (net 2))
 (segment (start 176.178612 103.349388) (end 179.96 99.568) (width 0.8) (layer F.Cu) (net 2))
 (segment (start 176.178612 103.678388) (end 176.178612 103.349388) (width 0.8) (layer F.Cu) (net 2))
 (segment (start 175.717 104.14) (end 176.178612 103.678388) (width 0.8) (layer F.Cu) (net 2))
 (segment (start 159.563 103.073) (end 159.512 103.124) (width 0.8) (layer F.Cu) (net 2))
 (segment (start 162.56 103.073) (end 159.563 103.073) (width 0.8) (layer F.Cu) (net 2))
 (segment (start 164.32001 97.989674) (end 164.32001 97.06) (width 0.8) (layer F.Cu) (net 2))
 (segment (start 164.32001 101.31299) (end 164.32001 97.989674) (width 0.8) (layer F.Cu) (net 2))
 (segment (start 162.56 103.073) (end 164.32001 101.31299) (width 0.8) (layer F.Cu) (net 2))
 (segment (start 141.678501 76.6575) (end 141.628001 76.708) (width 0.8) (layer F.Cu) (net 2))
 (segment (start 145.6975 76.6575) (end 141.678501 76.6575) (width 0.8) (layer F.Cu) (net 2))
 (segment (start 161.387388 86.008612) (end 161.387388 86.008612) (width 0.8) (layer F.Cu) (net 2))
 (segment (start 144.78 95.961) (end 144.78 92.084522) (width 0.8) (layer F.Cu) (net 2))
 (segment (start 156.96749 89.92749) (end 157.40751 89.92749) (width 0.8) (layer F.Cu) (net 2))
 (segment (start 159.96851 87.42749) (end 161.387388 86.008612) (width 0.8) (layer F.Cu) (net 2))
 (segment (start 158.757826 87.42749) (end 159.96851 87.42749) (width 0.8) (layer F.Cu) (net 2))
 (segment (start 158.37999 88.95501) (end 158.37999 87.805326) (width 0.8) (layer F.Cu) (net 2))
 (segment (start 157.40751 89.92749) (end 158.37999 88.95501) (width 0.8) (layer F.Cu) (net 2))
 (segment (start 158.37999 87.805326) (end 158.757826 87.42749) (width 0.8) (layer F.Cu) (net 2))
 (segment (start 154.13299 87.09299) (end 156.96749 89.92749) (width 0.8) (layer F.Cu) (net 2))
 (segment (start 161.387388 85.043612) (end 161.849 84.582) (width 0.8) (layer F.Cu) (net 2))
 (segment (start 149.771532 87.09299) (end 154.13299 87.09299) (width 0.8) (layer F.Cu) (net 2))
 (segment (start 144.78 92.084522) (end 149.771532 87.09299) (width 0.8) (layer F.Cu) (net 2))
 (segment (start 146.812 97.993) (end 144.78 95.961) (width 0.8) (layer F.Cu) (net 2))
 (segment (start 173.740612 95.203612) (end 175.595612 95.203612) (width 0.8) (layer F.Cu) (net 2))
 (segment (start 173.279 94.742) (end 173.740612 95.203612) (width 0.8) (layer F.Cu) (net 2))
 (via (at 171.196 87.63) (size 0.8) (drill 0.4) (layers F.Cu B.Cu) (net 2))
 (segment (start 171.704 87.122) (end 171.196 87.63) (width 0.25) (layer F.Cu) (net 2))
 (segment (start 171.704 85.725) (end 171.704 87.122) (width 0.25) (layer F.Cu) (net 2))
 (segment (start 171.196 87.63) (end 167.64 87.63) (width 0.25) (layer B.Cu) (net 2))
 (via (at 165.608 89.662) (size 0.8) (drill 0.4) (layers F.Cu B.Cu) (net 2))
 (segment (start 167.64 87.63) (end 165.608 89.662) (width 0.25) (layer B.Cu) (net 2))
 (segment (start 165.608 90.052) (end 165.5125 90.1475) (width 0.25) (layer F.Cu) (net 2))
 (segment (start 165.608 89.662) (end 165.608 90.052) (width 0.25) (layer F.Cu) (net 2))
 (segment (start 171.196 87.63) (end 171.196 90.678) (width 0.25) (layer B.Cu) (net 2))
 (segment (start 173.228 92.71) (end 173.2535 92.71) (width 0.25) (layer B.Cu) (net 2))
 (via (at 173.2535 92.71) (size 0.8) (drill 0.4) (layers F.Cu B.Cu) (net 2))
 (segment (start 171.196 90.678) (end 173.228 92.71) (width 0.25) (layer B.Cu) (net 2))
 (segment (start 173.2535 92.71) (end 173.2535 94.7165) (width 0.25) (layer B.Cu) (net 2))
 (via (at 173.279 94.742) (size 0.8) (drill 0.4) (layers F.Cu B.Cu) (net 2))
 (segment (start 173.2535 94.7165) (end 173.279 94.742) (width 0.25) (layer B.Cu) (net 2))
 (segment (start 161.387388 86.008612) (end 161.387388 85.043612) (width 0.8) (layer F.Cu) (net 2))
 (via (at 161.387388 86.008612) (size 0.8) (drill 0.4) (layers F.Cu B.Cu) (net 2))
 (segment (start 161.954612 86.008612) (end 165.608 89.662) (width 0.25) (layer B.Cu) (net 2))
 (segment (start 161.387388 86.008612) (end 161.954612 86.008612) (width 0.25) (layer B.Cu) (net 2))
 (segment (start 165.208001 90.061999) (end 165.208001 96.157999) (width 0.25) (layer B.Cu) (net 2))
 (segment (start 165.608 89.662) (end 165.208001 90.061999) (width 0.25) (layer B.Cu) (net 2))
 (segment (start 165.208001 96.157999) (end 164.338 97.028) (width 0.25) (layer B.Cu) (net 2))
 (via (at 164.338 97.028) (size 0.8) (drill 0.4) (layers F.Cu B.Cu) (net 2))
 (segment (start 161.985 104.648) (end 162.56 104.648) (width 0.25) (layer F.Cu) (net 29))
 (segment (start 158.766 104.648) (end 161.985 104.648) (width 0.25) (layer F.Cu) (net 29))
 (segment (start 158.242 104.124) (end 158.766 104.648) (width 0.25) (layer F.Cu) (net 29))
 (segment (start 158.242 103.124) (end 158.242 104.124) (width 0.25) (layer F.Cu) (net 29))
 (segment (start 161.1 97.820774) (end 161.1 97.06) (width 0.25) (layer F.Cu) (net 29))
 (segment (start 158.242 100.678774) (end 161.1 97.820774) (width 0.25) (layer F.Cu) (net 29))
 (segment (start 158.242 103.124) (end 158.242 100.678774) (width 0.25) (layer F.Cu) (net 29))
 (segment (start 171.704 81.347) (end 171.704 84.455) (width 0.25) (layer F.Cu) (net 38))
 (segment (start 171.704 80.772) (end 171.704 81.347) (width 0.25) (layer F.Cu) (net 38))
 (segment (start 171.704 83.900021) (end 171.115979 83.312) (width 0.25) (layer F.Cu) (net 38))
 (via (at 170.18 83.312) (size 0.8) (drill 0.4) (layers F.Cu B.Cu) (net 38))
 (segment (start 171.115979 83.312) (end 170.18 83.312) (width 0.25) (layer F.Cu) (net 38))
 (segment (start 171.704 84.455) (end 171.704 83.900021) (width 0.25) (layer F.Cu) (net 38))
 (segment (start 163.081159 83.286239) (end 157.226 89.141398) (width 0.25) (layer B.Cu) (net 38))
 (segment (start 168.272126 83.286239) (end 163.081159 83.286239) (width 0.25) (layer B.Cu) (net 38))
 (segment (start 168.297887 83.312) (end 168.272126 83.286239) (width 0.25) (layer B.Cu) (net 38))
 (segment (start 170.18 83.312) (end 168.297887 83.312) (width 0.25) (layer B.Cu) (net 38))
 (segment (start 157.226 89.141398) (end 157.226 93.218) (width 0.25) (layer B.Cu) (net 38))
 (via (at 158.496799 92.957038) (size 0.8) (drill 0.4) (layers F.Cu B.Cu) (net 38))
 (segment (start 158.235837 93.218) (end 158.496799 92.957038) (width 0.25) (layer B.Cu) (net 38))
 (segment (start 157.226 93.218) (end 158.235837 93.218) (width 0.25) (layer B.Cu) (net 38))
 (segment (start 158.306337 93.1475) (end 157.1875 93.1475) (width 0.25) (layer F.Cu) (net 38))
 (segment (start 158.496799 92.957038) (end 158.306337 93.1475) (width 0.25) (layer F.Cu) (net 38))
 (segment (start 157.166 92.126) (end 157.1875 92.1475) (width 0.25) (layer F.Cu) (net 5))
 (segment (start 152.314 92.126) (end 157.166 92.126) (width 0.25) (layer F.Cu) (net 5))
 (segment (start 151.892 91.704) (end 152.314 92.126) (width 0.25) (layer F.Cu) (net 5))
 (segment (start 151.892 88.138) (end 151.892 91.704) (width 0.25) (layer F.Cu) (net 5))
 (segment (start 154.385612 99.106388) (end 153.924 99.568) (width 0.25) (layer F.Cu) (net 1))
 (segment (start 154.69401 98.79799) (end 154.385612 99.106388) (width 0.25) (layer F.Cu) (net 1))
 (segment (start 154.69401 95.80349) (end 154.69401 98.79799) (width 0.25) (layer F.Cu) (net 1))
 (segment (start 156.35 94.1475) (end 154.69401 95.80349) (width 0.25) (layer F.Cu) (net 1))
 (segment (start 157.1875 94.1475) (end 156.35 94.1475) (width 0.25) (layer F.Cu) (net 1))
 (segment (start 153.924 99.568) (end 150.876 99.568) (width 0.25) (layer F.Cu) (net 1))
 (segment (start 150.876 99.568) (end 146.812 99.568) (width 0.25) (layer F.Cu) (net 1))
 (segment (start 149.86 93.472) (end 150.114 93.726) (width 0.25) (layer F.Cu) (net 4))
 (segment (start 146.812 93.472) (end 149.86 93.472) (width 0.25) (layer F.Cu) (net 4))
 (segment (start 156.35 92.6475) (end 157.1875 92.6475) (width 0.25) (layer F.Cu) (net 4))
 (segment (start 154.376499 94.621001) (end 156.35 92.6475) (width 0.25) (layer F.Cu) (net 4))
 (segment (start 150.159001 94.621001) (end 154.376499 94.621001) (width 0.25) (layer F.Cu) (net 4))
 (segment (start 150.114 94.576) (end 150.159001 94.621001) (width 0.25) (layer F.Cu) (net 4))
 (segment (start 150.114 93.726) (end 150.114 94.576) (width 0.25) (layer F.Cu) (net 4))
 (segment (start 175.514 99.06) (end 175.768 99.314) (width 0.25) (layer F.Cu) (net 42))
 (segment (start 173.228 99.06) (end 175.514 99.06) (width 0.25) (layer F.Cu) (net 42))
 (segment (start 176.830388 104.601612) (end 177.292 104.14) (width 0.25) (layer F.Cu) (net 43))
 (segment (start 176.52199 104.91001) (end 176.830388 104.601612) (width 0.25) (layer F.Cu) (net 43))
 (segment (start 172.77901 104.91001) (end 176.52199 104.91001) (width 0.25) (layer F.Cu) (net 43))
 (segment (start 172.263 104.394) (end 172.77901 104.91001) (width 0.25) (layer F.Cu) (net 43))
 (segment (start 169.164 86.279979) (end 169.164 85.725) (width 0.25) (layer F.Cu) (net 12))
 (segment (start 168.550218 86.893761) (end 169.164 86.279979) (width 0.25) (layer F.Cu) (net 12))
 (segment (start 167.202013 86.893761) (end 168.550218 86.893761) (width 0.25) (layer F.Cu) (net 12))
 (segment (start 164.328264 89.76751) (end 167.202013 86.893761) (width 0.25) (layer F.Cu) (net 12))
 (segment (start 163.371736 89.76751) (end 164.328264 89.76751) (width 0.25) (layer F.Cu) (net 12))
 (segment (start 163.1 89.495774) (end 163.371736 89.76751) (width 0.25) (layer F.Cu) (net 12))
 (segment (start 163.1 88.735) (end 163.1 89.495774) (width 0.25) (layer F.Cu) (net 12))
 (segment (start 164.32071 88.51429) (end 164.1 88.735) (width 0.25) (layer F.Cu) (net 14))
 (segment (start 167.973239 84.861761) (end 164.32071 88.51429) (width 0.25) (layer F.Cu) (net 14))
 (segment (start 168.757239 84.861761) (end 167.973239 84.861761) (width 0.25) (layer F.Cu) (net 14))
 (segment (start 169.164 84.455) (end 168.757239 84.861761) (width 0.25) (layer F.Cu) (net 14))
 (segment (start 170.434 86.279979) (end 170.434 85.725) (width 0.25) (layer F.Cu) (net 15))
 (segment (start 170.434 87.0635) (end 170.434 86.279979) (width 0.25) (layer F.Cu) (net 15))
 (segment (start 166.35 91.1475) (end 170.434 87.0635) (width 0.25) (layer F.Cu) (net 15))
 (segment (start 165.5125 91.1475) (end 166.35 91.1475) (width 0.25) (layer F.Cu) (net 15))
 (segment (start 171.653 98.485) (end 171.653 99.06) (width 0.25) (layer F.Cu) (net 20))
 (segment (start 166.8155 93.6475) (end 171.653 98.485) (width 0.25) (layer F.Cu) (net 20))
 (segment (start 165.5125 93.6475) (end 166.8155 93.6475) (width 0.25) (layer F.Cu) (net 20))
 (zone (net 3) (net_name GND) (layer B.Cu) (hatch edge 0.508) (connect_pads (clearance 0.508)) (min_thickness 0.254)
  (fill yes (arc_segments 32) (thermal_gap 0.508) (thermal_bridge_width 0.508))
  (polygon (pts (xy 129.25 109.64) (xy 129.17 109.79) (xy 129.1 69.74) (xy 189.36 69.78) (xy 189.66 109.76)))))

